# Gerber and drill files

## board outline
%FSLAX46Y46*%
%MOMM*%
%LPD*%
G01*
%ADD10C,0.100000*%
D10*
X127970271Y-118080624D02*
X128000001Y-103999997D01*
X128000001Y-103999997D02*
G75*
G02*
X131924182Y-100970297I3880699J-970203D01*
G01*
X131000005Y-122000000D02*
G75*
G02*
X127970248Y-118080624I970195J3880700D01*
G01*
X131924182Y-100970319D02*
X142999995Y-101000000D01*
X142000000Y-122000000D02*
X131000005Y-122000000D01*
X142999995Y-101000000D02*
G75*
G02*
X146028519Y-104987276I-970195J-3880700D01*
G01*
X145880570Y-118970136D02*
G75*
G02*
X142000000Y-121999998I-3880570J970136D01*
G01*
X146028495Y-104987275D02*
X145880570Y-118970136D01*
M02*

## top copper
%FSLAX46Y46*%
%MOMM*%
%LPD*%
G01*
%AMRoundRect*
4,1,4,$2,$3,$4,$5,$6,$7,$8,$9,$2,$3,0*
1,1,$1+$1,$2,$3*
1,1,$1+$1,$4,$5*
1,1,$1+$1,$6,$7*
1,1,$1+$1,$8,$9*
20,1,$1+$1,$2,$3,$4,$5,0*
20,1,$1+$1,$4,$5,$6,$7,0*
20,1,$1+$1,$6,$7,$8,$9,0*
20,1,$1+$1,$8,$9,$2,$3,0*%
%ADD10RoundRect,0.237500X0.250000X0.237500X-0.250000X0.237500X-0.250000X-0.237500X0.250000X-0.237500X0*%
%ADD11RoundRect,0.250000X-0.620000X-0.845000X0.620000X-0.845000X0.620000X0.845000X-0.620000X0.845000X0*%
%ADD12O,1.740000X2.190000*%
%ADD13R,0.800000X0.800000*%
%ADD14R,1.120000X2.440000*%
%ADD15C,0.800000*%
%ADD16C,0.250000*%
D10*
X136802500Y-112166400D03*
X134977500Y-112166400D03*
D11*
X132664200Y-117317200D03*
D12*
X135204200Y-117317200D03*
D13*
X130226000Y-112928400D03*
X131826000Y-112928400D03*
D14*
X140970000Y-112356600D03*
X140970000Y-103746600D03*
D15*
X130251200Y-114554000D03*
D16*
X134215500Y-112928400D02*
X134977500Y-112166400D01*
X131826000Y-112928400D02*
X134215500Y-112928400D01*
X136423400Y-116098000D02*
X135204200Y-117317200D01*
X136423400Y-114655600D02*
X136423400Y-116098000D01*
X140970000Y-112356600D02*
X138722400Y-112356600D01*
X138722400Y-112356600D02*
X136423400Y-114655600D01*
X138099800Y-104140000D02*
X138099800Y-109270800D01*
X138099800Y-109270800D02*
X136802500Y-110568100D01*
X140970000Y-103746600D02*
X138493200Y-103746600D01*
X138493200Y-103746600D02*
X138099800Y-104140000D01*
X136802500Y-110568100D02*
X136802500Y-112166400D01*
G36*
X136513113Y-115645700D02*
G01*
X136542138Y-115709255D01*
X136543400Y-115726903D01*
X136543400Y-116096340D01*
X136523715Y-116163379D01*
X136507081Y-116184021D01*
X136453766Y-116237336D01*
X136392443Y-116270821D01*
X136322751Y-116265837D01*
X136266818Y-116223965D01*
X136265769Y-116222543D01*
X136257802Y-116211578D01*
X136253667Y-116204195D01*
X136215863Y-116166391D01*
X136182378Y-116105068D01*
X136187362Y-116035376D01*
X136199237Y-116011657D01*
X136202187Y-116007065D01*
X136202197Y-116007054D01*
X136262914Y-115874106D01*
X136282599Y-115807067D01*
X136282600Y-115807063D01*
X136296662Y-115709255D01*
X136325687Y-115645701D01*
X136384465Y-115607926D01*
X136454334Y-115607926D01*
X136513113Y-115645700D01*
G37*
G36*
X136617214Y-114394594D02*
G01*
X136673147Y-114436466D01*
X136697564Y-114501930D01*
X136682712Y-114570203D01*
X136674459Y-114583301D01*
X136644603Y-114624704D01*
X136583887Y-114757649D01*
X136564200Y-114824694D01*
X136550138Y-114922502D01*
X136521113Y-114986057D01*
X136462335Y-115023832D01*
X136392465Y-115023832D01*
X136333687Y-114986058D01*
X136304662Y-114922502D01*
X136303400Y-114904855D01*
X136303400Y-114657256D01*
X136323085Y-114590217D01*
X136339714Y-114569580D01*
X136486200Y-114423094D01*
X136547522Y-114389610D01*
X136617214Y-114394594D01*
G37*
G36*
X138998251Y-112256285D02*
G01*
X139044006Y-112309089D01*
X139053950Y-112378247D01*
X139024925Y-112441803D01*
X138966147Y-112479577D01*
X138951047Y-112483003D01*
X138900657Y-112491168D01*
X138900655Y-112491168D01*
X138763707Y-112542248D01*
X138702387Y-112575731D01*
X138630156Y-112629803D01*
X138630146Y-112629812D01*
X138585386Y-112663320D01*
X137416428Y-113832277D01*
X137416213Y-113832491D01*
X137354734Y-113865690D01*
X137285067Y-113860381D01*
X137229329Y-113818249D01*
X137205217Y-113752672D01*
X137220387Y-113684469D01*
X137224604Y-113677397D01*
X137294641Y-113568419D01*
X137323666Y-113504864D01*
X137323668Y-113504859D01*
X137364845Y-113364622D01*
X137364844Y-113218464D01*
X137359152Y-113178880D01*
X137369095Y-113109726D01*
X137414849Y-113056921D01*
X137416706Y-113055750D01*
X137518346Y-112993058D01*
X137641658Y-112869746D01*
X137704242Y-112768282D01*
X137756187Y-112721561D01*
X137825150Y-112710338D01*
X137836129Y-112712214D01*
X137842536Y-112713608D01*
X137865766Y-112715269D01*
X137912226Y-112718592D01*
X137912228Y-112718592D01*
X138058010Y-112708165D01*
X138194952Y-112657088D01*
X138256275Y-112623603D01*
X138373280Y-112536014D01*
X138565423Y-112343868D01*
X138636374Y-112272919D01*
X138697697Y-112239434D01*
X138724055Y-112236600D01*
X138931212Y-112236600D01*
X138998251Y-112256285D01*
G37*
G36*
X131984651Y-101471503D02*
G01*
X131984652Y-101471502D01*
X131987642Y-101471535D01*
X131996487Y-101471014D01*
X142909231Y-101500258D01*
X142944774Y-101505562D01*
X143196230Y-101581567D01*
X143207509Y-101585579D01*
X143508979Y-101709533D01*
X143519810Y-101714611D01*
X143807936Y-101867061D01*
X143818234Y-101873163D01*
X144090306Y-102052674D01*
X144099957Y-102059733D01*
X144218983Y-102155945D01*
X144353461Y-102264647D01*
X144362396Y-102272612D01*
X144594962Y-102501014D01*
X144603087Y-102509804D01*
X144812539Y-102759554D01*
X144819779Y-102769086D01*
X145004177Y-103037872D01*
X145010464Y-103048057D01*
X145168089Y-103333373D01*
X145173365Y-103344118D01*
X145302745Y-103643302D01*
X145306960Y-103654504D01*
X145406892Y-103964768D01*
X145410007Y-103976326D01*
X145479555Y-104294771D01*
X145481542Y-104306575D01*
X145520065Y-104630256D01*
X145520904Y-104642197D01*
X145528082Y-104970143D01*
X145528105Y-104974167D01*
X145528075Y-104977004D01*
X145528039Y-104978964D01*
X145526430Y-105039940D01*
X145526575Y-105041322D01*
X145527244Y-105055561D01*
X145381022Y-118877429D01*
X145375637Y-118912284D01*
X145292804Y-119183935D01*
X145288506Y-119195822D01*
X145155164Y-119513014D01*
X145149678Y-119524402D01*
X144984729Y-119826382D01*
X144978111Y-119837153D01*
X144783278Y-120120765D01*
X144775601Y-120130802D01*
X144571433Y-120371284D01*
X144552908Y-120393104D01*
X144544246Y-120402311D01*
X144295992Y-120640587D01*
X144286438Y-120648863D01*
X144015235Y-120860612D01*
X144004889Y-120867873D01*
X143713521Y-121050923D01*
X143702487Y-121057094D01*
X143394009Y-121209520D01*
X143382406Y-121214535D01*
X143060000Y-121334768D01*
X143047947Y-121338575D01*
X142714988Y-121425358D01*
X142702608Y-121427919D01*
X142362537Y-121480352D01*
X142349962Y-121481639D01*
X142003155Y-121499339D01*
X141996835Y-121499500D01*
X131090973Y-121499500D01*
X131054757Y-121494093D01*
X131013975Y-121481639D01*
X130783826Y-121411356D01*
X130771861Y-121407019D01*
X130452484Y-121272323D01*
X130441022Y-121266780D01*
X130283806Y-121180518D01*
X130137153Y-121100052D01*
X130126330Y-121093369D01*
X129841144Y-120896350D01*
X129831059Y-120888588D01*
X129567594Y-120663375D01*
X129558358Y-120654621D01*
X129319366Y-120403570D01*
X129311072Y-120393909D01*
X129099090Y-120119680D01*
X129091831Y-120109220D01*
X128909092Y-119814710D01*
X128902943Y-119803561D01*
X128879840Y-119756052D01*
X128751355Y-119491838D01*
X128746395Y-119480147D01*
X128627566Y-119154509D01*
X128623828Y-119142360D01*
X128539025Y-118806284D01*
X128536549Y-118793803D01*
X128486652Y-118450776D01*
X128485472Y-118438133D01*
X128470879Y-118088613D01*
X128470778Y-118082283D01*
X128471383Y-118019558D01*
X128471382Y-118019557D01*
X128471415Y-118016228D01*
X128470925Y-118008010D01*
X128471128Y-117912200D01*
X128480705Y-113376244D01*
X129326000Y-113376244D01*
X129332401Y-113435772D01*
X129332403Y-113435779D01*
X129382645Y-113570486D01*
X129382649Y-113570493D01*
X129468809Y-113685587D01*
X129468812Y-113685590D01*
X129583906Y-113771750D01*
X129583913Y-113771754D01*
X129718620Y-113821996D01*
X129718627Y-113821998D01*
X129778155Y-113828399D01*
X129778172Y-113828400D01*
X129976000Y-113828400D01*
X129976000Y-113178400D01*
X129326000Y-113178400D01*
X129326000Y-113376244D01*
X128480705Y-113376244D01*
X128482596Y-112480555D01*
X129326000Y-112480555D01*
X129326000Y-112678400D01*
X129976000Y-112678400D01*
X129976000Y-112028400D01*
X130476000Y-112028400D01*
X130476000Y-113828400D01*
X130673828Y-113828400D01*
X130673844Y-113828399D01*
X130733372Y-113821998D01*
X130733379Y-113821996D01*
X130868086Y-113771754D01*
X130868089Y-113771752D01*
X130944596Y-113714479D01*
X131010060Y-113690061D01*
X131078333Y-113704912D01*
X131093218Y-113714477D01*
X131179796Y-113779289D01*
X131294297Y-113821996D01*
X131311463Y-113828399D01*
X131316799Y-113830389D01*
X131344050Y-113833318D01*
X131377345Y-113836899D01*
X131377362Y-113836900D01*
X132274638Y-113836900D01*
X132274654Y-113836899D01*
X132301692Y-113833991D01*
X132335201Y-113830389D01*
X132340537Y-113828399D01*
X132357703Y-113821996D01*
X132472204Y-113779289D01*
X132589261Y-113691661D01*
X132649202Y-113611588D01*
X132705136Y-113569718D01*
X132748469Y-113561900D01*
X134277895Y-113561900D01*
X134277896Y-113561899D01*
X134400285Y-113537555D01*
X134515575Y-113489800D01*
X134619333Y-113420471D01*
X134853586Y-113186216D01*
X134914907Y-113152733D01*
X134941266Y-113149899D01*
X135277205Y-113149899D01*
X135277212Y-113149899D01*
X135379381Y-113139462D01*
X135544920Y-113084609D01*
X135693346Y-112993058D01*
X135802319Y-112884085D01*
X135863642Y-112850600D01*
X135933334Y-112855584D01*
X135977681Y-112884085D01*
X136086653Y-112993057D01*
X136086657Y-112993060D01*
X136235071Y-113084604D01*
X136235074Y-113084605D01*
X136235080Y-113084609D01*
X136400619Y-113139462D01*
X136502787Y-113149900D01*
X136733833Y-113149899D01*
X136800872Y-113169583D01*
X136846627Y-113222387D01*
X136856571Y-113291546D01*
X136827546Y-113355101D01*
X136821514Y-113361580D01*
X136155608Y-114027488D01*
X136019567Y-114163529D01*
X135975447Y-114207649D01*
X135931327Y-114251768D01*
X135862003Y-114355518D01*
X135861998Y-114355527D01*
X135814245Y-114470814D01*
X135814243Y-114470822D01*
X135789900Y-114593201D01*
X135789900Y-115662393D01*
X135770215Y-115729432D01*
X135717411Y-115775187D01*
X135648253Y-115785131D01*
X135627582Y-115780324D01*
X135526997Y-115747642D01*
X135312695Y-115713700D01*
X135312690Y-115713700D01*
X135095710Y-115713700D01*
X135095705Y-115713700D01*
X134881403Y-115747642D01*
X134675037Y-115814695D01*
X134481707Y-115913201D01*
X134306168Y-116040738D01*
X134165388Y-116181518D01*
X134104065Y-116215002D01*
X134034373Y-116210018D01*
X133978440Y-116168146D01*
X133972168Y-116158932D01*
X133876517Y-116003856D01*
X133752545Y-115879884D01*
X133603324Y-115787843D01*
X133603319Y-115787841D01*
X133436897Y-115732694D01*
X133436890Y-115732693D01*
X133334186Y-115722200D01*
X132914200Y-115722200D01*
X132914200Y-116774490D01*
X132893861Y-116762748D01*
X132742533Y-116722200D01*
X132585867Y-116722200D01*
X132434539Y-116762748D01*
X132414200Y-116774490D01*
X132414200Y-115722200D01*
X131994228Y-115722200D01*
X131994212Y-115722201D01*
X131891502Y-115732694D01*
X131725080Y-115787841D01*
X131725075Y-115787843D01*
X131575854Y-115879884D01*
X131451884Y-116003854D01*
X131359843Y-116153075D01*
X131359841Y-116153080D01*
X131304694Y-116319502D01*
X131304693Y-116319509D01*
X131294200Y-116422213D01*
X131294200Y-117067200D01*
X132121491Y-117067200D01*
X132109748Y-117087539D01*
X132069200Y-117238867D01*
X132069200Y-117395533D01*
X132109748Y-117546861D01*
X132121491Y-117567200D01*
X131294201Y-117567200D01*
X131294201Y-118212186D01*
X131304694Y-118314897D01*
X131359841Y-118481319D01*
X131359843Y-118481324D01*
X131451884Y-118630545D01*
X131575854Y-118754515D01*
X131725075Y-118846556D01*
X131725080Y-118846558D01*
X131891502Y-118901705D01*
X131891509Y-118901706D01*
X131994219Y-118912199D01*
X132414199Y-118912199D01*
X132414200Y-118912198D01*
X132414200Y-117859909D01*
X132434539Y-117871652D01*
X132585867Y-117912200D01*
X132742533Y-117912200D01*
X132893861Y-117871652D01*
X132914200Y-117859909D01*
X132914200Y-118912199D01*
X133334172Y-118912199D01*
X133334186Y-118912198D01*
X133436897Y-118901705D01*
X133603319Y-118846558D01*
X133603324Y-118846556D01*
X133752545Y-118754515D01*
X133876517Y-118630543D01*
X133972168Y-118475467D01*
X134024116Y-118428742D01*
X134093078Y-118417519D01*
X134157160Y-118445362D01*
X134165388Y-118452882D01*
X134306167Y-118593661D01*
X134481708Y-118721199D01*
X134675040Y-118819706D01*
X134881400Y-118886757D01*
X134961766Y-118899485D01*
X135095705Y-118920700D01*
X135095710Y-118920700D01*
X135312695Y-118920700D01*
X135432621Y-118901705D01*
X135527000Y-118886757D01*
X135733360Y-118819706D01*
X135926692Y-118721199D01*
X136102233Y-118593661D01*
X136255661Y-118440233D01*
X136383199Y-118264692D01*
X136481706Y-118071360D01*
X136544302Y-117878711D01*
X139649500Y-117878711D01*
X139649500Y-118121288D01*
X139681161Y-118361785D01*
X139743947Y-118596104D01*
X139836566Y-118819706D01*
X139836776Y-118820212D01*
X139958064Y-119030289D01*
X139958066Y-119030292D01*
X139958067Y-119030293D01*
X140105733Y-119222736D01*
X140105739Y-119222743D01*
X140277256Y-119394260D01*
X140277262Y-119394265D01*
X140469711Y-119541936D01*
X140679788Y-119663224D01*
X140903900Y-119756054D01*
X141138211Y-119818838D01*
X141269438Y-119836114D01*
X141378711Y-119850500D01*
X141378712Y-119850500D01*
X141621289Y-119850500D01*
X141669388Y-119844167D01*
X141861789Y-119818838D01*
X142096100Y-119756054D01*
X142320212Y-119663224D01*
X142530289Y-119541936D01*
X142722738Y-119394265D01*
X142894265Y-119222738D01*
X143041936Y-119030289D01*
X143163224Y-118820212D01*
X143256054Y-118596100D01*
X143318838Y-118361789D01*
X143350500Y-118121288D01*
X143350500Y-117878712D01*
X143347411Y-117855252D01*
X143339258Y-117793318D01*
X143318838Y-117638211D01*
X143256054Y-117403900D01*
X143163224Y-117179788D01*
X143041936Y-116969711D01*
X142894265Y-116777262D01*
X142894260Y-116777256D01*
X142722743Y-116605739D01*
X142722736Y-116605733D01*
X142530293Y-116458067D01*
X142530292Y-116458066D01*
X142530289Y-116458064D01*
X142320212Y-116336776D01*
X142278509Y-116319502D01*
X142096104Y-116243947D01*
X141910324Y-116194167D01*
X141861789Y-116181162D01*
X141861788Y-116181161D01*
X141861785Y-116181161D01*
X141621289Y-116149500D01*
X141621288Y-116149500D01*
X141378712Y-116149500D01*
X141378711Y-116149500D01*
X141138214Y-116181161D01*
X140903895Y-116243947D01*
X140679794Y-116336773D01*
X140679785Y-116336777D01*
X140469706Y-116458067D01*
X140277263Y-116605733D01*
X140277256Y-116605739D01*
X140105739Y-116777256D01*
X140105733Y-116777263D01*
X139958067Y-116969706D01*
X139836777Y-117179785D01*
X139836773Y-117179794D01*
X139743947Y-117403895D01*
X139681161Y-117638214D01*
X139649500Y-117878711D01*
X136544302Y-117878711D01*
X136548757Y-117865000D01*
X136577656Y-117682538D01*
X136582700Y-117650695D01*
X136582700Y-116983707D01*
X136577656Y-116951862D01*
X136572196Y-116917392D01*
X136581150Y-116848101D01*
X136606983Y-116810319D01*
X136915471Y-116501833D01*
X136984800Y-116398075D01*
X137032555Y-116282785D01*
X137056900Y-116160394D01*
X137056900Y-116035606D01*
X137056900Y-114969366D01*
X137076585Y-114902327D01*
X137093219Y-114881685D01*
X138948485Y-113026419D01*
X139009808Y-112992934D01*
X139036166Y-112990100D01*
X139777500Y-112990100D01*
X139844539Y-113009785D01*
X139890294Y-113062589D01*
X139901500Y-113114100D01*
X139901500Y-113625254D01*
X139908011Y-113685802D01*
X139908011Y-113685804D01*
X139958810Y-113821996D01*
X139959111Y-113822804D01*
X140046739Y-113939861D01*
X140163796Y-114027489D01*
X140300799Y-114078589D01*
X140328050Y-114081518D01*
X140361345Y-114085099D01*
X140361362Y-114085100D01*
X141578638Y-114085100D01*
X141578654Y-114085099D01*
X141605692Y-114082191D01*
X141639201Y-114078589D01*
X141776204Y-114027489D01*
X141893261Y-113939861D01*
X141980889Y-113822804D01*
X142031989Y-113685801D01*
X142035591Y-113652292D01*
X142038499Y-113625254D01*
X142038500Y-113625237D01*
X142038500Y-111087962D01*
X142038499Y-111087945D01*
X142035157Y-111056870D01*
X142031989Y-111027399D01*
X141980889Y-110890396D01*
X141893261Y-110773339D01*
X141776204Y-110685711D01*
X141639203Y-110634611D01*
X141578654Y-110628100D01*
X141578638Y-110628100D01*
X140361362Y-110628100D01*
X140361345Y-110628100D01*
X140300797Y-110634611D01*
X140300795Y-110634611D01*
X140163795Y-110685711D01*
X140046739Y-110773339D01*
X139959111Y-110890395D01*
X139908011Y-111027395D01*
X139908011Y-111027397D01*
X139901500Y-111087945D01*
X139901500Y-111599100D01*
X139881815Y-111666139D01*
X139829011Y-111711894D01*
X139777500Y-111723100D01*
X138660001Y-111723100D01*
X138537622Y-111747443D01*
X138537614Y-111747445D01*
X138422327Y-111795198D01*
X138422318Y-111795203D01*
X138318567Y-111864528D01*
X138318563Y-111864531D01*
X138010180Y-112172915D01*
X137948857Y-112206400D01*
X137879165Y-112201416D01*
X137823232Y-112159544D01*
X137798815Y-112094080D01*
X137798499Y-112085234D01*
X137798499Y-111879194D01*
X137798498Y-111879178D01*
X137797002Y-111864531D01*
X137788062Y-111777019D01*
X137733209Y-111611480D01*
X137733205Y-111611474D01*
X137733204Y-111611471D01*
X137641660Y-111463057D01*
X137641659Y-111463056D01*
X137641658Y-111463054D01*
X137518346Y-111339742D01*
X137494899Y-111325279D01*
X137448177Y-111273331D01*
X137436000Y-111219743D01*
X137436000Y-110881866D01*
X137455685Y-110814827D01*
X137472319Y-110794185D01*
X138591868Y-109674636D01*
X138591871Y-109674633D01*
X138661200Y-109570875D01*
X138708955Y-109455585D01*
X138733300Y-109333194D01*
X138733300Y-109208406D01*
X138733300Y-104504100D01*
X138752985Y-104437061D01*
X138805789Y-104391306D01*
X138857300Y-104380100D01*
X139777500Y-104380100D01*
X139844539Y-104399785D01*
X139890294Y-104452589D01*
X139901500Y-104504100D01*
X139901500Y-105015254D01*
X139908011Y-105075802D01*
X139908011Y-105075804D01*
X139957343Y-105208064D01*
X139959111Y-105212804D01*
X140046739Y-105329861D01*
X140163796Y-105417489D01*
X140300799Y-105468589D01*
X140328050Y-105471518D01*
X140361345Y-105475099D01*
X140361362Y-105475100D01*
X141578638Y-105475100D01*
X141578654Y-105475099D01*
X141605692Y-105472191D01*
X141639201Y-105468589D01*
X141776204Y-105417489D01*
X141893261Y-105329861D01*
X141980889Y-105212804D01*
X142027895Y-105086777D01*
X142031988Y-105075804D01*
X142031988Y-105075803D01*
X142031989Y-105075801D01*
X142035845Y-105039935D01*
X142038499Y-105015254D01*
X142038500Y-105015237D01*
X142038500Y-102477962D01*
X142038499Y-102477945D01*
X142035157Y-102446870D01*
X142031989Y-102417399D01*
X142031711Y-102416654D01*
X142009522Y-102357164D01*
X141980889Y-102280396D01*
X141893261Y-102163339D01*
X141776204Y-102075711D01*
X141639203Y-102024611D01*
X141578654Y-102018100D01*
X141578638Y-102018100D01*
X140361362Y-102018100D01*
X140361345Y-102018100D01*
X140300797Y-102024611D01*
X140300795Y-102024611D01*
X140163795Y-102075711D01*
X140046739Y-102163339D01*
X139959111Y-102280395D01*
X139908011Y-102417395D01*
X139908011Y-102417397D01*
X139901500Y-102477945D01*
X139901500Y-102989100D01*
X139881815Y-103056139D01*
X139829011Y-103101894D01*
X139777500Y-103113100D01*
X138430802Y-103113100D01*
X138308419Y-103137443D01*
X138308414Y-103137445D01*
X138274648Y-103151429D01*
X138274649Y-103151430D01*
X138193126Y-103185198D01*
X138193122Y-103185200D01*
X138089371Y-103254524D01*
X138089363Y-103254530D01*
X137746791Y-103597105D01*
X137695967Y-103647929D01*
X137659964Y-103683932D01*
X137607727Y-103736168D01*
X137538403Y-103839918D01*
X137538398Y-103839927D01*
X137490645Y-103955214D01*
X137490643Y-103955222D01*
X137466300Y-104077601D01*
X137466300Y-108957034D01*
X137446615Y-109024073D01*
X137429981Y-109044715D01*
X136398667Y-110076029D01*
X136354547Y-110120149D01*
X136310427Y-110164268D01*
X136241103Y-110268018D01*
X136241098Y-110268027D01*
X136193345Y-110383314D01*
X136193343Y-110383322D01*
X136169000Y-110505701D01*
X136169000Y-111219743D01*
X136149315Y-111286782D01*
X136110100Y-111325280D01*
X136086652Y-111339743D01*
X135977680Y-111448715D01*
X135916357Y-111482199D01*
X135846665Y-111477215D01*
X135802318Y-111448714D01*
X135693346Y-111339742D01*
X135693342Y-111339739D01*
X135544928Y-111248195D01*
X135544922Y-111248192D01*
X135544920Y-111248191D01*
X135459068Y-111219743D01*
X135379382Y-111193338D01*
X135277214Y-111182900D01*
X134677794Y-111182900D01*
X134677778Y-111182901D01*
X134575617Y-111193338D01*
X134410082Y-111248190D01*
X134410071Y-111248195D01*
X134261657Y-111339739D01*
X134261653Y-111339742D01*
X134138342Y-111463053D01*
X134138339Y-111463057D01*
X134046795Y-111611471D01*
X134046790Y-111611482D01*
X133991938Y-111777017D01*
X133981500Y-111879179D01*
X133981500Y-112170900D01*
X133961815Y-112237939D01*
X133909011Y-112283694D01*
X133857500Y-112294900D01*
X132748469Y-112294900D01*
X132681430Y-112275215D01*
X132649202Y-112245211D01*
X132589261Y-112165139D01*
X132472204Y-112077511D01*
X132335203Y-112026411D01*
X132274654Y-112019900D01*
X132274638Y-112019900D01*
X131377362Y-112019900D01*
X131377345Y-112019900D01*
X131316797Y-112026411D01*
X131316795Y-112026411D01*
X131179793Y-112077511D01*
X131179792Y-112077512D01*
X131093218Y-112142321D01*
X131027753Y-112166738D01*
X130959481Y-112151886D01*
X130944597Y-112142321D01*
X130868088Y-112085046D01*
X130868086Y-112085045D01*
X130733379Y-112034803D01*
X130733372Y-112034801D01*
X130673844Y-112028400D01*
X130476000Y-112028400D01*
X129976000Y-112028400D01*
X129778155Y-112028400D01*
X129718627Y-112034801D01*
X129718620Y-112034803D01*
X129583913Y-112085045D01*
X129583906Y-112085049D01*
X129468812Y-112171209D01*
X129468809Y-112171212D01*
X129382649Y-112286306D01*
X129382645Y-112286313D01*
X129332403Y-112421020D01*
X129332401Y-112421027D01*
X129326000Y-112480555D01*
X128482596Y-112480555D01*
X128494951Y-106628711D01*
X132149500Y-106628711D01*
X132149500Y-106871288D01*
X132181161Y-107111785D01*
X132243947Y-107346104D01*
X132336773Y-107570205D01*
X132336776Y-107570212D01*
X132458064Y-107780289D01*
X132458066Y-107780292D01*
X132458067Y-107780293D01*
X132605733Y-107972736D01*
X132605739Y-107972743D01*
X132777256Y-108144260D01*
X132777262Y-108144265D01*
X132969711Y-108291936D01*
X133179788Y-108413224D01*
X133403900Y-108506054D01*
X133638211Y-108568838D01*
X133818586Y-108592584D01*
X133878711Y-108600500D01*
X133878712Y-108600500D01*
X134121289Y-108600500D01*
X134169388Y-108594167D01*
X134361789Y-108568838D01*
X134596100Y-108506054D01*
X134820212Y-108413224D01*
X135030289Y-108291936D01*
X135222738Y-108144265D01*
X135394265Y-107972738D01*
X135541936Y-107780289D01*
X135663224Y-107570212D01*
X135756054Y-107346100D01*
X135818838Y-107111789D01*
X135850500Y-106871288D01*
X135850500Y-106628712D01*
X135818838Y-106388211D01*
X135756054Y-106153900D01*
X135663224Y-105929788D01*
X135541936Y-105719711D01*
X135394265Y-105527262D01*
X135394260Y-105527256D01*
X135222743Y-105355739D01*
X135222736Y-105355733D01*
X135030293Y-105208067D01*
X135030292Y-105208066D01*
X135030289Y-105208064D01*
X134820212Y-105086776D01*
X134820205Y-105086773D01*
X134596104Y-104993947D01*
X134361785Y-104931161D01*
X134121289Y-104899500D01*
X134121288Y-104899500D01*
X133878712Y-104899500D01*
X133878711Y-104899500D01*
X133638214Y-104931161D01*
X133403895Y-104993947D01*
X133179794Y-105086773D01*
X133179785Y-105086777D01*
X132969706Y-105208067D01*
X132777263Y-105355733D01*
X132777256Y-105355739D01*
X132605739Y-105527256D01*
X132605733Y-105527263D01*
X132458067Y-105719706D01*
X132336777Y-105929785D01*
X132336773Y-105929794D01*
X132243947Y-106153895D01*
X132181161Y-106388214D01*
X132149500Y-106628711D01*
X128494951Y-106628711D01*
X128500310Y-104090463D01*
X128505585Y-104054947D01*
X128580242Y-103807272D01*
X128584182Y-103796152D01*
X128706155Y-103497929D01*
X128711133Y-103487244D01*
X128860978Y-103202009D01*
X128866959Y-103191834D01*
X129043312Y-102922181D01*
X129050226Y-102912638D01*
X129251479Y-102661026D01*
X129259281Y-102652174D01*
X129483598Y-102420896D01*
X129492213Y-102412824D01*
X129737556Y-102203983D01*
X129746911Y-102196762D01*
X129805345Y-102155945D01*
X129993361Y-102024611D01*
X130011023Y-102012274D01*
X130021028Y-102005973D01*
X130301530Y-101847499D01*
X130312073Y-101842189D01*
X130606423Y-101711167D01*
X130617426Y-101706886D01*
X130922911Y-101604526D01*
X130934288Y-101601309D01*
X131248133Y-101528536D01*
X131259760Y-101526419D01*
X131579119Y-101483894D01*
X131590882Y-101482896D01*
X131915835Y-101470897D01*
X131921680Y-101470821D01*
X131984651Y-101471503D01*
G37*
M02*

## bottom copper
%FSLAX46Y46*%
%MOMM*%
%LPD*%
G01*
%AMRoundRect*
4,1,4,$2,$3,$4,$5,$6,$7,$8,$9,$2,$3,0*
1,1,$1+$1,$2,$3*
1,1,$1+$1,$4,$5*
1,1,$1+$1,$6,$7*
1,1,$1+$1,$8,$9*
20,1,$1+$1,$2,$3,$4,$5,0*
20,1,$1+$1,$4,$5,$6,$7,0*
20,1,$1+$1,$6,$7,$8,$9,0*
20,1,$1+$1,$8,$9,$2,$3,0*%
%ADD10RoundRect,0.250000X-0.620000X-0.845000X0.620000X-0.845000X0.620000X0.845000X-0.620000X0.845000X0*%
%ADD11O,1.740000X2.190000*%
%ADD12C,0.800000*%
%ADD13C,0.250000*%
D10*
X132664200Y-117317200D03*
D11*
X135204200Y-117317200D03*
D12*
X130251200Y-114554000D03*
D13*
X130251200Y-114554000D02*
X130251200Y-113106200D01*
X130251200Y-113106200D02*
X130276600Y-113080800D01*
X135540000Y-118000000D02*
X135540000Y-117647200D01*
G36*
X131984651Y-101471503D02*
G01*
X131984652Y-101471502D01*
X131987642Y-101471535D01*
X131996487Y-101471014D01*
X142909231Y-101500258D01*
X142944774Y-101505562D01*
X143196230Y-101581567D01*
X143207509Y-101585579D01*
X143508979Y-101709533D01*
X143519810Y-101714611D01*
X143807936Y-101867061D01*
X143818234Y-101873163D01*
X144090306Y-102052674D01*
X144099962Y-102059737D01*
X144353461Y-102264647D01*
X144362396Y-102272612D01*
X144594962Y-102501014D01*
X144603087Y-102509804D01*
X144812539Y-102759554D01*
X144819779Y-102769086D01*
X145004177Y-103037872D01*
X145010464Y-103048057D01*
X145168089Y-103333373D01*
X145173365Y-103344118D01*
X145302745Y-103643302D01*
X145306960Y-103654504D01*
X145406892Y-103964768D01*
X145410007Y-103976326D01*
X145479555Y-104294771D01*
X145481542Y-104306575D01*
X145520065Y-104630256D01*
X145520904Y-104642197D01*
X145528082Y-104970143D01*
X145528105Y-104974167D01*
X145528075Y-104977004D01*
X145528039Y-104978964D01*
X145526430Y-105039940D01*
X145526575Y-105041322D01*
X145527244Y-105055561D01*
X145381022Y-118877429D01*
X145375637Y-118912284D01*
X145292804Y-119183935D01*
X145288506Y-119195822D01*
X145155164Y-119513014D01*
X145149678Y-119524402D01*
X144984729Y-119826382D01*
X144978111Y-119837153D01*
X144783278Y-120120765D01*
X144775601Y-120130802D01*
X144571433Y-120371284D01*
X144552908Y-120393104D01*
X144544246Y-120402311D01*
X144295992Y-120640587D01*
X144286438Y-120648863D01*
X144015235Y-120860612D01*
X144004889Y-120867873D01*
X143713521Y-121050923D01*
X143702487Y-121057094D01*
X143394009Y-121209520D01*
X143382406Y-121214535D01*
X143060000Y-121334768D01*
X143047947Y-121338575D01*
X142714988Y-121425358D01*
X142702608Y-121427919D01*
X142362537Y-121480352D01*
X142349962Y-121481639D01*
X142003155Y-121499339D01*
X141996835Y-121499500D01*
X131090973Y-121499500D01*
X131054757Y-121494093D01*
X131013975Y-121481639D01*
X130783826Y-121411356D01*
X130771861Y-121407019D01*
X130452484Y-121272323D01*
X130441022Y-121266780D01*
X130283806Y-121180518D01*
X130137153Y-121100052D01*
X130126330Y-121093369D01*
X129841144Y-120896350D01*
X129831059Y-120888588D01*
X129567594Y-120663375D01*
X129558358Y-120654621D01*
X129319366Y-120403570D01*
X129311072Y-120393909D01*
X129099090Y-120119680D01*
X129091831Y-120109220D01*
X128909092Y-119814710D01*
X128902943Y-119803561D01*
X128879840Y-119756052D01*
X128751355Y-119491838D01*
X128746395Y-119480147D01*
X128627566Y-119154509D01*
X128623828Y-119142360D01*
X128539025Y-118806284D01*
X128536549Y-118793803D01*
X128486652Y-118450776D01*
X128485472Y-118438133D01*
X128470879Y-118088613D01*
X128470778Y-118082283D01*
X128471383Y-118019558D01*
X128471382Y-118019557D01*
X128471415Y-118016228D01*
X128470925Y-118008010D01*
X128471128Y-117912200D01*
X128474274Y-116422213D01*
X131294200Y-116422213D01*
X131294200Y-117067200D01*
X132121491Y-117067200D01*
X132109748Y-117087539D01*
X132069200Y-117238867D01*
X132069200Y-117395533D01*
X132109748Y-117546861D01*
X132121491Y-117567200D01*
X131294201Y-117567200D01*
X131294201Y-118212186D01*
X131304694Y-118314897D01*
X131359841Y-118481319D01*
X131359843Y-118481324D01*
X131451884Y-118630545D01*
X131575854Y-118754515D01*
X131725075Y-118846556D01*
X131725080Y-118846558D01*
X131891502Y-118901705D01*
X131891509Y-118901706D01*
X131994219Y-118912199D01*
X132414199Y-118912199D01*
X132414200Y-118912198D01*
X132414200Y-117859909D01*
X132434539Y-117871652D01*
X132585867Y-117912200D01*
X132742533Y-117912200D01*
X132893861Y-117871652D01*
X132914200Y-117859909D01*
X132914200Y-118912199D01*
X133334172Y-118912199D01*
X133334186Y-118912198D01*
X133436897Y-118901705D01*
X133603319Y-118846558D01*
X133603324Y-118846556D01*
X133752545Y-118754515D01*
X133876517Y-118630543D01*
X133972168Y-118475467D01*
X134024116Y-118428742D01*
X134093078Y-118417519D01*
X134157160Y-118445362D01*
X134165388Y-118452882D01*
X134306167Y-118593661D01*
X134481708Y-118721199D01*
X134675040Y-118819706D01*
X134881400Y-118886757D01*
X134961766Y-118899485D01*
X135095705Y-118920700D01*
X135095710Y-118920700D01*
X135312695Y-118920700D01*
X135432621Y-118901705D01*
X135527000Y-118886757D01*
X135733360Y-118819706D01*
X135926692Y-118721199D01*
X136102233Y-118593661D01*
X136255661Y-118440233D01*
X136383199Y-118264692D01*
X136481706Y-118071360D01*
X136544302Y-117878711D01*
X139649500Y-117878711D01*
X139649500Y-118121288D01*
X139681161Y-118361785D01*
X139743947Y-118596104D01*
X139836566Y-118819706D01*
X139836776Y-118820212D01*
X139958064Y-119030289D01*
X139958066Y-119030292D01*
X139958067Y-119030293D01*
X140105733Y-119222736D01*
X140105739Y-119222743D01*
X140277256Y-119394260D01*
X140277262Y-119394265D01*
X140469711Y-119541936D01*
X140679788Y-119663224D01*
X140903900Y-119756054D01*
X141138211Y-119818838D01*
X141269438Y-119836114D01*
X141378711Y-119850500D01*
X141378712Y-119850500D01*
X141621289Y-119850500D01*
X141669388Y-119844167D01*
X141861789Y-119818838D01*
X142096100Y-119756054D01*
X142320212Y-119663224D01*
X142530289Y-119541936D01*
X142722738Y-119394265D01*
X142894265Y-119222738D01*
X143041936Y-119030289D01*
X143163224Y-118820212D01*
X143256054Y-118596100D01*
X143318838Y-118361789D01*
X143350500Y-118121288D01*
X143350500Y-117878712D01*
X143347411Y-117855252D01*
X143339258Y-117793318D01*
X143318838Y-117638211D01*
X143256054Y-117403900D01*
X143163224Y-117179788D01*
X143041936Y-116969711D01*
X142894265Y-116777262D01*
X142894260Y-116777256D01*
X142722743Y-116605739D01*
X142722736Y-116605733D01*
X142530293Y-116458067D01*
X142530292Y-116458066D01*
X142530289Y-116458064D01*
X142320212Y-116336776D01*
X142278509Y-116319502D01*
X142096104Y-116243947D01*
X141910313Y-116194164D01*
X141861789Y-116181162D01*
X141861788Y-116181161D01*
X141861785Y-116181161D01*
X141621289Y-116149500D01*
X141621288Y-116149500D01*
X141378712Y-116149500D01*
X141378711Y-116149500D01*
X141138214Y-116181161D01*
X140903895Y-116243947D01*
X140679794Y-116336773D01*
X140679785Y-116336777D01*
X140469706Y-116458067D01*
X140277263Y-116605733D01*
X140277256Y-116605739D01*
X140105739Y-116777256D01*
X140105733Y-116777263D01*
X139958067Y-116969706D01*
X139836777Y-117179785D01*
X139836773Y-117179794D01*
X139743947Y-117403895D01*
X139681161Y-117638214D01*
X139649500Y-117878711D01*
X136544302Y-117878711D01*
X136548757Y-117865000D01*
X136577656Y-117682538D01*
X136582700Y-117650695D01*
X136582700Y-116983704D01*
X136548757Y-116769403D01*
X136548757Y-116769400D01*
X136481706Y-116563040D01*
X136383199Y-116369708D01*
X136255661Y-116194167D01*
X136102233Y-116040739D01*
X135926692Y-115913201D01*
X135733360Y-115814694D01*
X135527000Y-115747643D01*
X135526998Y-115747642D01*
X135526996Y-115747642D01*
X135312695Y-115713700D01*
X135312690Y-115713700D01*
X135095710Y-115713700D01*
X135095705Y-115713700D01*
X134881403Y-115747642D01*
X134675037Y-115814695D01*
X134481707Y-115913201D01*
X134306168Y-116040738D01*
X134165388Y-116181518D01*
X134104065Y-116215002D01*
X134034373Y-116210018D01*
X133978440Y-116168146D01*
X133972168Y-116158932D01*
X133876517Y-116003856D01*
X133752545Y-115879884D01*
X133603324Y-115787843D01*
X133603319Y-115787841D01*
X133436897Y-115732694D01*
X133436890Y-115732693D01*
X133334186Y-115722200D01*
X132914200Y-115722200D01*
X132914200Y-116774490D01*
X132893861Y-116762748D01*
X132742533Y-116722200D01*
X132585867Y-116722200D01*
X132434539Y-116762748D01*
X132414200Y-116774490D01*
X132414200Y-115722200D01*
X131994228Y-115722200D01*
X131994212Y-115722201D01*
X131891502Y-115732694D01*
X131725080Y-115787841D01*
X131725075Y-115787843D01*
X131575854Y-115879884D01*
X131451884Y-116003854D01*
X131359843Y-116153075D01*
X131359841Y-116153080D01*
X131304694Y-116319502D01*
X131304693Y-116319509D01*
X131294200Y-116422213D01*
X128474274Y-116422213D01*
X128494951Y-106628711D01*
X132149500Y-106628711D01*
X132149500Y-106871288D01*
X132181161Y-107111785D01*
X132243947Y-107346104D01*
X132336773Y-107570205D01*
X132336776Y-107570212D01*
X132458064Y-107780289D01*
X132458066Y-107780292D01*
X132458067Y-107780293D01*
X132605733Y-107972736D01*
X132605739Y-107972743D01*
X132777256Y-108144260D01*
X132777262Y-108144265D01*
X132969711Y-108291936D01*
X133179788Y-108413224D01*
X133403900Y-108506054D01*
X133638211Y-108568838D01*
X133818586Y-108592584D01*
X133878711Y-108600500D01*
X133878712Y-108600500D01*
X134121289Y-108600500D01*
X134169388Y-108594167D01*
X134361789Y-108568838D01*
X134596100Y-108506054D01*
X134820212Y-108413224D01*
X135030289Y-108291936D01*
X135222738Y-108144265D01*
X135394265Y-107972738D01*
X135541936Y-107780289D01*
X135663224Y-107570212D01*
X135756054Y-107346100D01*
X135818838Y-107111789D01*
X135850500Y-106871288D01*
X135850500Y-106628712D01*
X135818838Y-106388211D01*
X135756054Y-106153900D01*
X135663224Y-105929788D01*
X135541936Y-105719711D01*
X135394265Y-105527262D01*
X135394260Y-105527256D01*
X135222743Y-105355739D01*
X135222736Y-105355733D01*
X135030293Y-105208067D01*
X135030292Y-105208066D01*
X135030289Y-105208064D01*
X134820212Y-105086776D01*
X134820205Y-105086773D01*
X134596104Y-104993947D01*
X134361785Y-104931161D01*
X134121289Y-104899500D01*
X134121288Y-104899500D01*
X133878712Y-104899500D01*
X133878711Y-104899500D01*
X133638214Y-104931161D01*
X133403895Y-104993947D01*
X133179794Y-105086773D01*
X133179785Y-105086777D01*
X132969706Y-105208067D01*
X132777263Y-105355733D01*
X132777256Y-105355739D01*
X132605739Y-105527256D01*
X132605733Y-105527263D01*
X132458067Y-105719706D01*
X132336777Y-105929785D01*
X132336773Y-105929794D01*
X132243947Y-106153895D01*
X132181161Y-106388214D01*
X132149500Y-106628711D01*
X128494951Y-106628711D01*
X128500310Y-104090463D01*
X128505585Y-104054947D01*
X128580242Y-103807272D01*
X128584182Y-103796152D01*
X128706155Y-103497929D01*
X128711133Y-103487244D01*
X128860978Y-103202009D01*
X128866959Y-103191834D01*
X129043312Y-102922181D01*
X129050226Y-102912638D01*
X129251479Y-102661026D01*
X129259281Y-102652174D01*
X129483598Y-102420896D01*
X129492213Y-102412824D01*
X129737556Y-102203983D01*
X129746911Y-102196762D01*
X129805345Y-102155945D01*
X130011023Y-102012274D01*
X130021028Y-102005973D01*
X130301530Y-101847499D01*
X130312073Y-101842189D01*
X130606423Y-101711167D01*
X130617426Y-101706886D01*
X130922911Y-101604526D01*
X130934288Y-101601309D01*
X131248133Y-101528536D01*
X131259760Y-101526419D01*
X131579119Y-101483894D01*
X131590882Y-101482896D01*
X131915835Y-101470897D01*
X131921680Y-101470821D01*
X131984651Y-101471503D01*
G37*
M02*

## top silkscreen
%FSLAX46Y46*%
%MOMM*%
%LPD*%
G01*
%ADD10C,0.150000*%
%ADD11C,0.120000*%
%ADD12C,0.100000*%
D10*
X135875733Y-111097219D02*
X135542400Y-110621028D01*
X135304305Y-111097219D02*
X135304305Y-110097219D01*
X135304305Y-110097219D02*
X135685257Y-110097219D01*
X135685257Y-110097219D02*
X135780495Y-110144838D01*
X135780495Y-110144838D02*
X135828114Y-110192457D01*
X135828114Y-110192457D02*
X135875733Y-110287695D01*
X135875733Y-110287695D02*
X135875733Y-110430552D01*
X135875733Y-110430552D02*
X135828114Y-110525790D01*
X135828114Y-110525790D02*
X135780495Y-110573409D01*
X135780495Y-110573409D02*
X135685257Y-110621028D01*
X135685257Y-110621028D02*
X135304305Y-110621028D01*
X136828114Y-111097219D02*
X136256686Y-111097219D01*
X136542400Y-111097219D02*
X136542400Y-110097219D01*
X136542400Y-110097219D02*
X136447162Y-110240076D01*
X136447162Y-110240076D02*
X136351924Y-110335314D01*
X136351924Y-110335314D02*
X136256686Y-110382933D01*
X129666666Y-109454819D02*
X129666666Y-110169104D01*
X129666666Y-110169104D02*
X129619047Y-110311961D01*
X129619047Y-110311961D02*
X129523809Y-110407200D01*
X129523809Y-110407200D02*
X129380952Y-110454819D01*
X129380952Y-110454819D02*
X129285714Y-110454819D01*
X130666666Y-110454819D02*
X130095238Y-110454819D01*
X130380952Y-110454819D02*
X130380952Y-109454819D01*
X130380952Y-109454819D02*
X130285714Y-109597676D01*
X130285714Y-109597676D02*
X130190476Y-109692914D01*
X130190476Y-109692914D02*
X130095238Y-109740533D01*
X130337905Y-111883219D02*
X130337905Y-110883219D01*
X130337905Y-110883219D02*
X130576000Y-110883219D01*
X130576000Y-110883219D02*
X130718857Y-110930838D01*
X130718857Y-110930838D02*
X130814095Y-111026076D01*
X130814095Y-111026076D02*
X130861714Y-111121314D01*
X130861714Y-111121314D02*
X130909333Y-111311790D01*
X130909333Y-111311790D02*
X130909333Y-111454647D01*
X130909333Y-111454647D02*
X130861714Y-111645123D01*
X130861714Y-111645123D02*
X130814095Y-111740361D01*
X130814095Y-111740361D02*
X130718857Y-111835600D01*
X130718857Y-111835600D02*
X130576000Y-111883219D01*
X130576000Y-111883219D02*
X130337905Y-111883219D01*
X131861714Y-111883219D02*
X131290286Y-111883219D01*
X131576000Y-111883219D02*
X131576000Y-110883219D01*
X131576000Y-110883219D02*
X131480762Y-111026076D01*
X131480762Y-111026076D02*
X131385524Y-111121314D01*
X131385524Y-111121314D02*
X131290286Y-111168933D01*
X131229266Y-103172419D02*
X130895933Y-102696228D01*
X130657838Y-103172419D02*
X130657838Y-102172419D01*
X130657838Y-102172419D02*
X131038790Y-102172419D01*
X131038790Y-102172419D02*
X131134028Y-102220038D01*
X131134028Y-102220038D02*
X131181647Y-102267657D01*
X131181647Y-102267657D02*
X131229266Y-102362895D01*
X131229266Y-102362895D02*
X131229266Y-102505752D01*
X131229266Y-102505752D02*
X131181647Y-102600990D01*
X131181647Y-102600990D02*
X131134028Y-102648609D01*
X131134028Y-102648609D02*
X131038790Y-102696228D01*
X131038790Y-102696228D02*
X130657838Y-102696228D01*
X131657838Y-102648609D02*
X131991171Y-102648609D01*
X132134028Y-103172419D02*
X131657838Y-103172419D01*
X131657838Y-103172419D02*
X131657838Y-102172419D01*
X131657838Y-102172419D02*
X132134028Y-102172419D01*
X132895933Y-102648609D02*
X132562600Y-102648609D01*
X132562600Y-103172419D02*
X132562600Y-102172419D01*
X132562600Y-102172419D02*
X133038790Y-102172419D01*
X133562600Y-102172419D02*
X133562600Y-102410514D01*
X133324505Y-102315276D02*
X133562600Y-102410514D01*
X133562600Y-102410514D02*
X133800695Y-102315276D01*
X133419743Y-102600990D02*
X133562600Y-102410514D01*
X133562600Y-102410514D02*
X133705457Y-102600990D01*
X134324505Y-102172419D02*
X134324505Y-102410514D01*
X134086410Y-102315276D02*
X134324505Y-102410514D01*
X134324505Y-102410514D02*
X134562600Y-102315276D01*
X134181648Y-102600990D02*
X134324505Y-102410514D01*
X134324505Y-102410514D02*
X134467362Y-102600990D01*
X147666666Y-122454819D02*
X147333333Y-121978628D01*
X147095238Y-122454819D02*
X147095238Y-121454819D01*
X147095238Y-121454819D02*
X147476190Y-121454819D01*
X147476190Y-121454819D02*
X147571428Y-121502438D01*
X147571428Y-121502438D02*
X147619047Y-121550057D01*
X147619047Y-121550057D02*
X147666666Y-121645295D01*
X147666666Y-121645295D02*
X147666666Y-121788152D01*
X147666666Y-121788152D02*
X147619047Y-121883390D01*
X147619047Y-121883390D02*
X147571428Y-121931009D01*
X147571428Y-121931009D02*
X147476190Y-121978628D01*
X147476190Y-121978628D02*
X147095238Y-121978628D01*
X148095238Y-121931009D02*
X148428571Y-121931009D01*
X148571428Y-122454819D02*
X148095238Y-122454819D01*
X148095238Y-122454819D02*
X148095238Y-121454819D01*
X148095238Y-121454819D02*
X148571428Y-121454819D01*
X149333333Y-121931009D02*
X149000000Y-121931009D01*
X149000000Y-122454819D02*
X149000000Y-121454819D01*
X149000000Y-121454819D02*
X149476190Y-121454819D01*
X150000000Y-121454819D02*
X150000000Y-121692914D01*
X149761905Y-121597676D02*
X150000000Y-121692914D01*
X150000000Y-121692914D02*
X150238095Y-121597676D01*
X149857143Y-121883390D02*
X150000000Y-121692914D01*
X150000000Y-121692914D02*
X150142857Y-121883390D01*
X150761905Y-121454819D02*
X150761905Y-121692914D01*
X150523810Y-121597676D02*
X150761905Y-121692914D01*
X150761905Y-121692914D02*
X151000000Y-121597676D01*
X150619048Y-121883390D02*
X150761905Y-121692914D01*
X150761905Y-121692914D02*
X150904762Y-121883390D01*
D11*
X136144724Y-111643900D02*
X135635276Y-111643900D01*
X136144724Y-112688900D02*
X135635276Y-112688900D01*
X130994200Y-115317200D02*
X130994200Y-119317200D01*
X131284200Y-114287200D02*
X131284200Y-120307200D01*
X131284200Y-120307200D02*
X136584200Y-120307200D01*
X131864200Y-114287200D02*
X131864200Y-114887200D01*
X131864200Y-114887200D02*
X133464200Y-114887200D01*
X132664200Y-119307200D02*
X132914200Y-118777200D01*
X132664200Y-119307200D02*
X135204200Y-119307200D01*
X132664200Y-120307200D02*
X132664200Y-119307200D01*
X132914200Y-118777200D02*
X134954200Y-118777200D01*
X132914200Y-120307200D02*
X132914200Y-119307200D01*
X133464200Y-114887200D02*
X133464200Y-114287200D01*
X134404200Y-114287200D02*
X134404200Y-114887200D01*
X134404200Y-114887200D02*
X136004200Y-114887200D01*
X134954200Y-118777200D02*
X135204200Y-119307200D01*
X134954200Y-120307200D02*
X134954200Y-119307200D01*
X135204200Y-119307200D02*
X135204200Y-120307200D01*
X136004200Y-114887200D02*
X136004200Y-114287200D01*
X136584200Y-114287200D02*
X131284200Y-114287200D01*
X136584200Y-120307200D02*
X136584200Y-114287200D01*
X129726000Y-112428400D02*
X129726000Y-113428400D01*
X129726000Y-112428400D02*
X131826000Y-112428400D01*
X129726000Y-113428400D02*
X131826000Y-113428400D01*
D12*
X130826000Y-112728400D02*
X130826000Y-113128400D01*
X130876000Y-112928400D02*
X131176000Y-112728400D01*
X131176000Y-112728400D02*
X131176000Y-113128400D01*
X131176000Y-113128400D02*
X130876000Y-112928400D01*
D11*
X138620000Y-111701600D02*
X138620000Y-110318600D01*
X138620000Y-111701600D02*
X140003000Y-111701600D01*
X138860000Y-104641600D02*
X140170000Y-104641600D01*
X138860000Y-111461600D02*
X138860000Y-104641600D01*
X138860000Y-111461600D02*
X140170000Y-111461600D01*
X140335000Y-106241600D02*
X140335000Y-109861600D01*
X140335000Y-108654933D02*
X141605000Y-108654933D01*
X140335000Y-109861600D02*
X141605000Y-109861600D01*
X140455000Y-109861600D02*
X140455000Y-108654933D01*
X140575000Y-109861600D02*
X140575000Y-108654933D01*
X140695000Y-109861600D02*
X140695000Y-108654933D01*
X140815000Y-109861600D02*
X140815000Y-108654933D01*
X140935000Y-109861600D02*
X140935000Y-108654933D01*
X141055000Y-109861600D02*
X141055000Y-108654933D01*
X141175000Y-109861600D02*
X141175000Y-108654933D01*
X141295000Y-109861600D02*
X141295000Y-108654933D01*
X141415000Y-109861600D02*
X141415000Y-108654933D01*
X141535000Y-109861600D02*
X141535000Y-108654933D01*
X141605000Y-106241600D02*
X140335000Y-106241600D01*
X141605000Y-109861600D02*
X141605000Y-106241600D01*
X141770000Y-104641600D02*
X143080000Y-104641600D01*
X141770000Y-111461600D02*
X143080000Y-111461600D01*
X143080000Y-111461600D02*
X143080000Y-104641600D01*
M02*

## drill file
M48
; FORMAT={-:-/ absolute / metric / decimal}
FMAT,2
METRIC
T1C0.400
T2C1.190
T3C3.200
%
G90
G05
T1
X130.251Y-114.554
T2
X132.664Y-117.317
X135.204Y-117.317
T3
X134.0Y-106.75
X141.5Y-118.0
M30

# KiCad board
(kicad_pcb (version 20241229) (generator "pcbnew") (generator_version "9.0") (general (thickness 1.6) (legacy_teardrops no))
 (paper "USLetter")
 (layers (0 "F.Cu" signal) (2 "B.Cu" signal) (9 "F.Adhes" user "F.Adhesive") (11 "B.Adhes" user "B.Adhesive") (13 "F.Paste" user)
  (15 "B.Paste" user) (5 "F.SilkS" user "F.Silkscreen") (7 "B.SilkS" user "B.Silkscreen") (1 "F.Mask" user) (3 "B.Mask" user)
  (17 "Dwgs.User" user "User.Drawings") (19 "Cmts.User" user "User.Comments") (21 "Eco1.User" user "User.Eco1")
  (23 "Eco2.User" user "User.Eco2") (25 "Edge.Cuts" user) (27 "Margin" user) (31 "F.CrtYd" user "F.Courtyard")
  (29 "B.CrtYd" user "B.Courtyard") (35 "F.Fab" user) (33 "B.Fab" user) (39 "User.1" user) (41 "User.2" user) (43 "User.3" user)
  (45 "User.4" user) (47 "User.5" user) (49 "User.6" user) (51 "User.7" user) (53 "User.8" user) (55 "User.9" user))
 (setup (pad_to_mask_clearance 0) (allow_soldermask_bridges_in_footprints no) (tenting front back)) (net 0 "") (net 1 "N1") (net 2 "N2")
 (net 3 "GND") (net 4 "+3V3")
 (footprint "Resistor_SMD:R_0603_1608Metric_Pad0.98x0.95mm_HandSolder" (layer "F.Cu") (at 135.89 112.1664 180)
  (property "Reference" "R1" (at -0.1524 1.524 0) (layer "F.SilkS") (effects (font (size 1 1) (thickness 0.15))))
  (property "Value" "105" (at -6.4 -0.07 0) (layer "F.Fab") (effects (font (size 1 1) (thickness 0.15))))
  (fp_line (start -0.254724 0.5225) (end 0.254724 0.5225) (stroke (width 0.12) (type solid)) (layer "F.SilkS"))
  (fp_line (start -0.254724 -0.5225) (end 0.254724 -0.5225) (stroke (width 0.12) (type solid)) (layer "F.SilkS"))
  (pad "1" smd roundrect (at -0.9125 0 180) (size 0.975 0.95) (layers "F.Cu" "F.Mask" "F.Paste") (roundrect_rratio 0.25) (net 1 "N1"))
  (pad "2" smd roundrect (at 0.9125 0 180) (size 0.975 0.95) (layers "F.Cu" "F.Mask" "F.Paste") (roundrect_rratio 0.25) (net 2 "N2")))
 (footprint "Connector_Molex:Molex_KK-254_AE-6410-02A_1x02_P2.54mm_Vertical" (layer "F.Cu") (at 132.6642 117.3172)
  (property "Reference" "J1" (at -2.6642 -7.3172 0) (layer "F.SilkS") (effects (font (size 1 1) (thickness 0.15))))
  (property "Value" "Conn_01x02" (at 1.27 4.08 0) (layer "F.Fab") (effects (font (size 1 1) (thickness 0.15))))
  (fp_line (start -1.67 -2) (end -1.67 2) (stroke (width 0.12) (type solid)) (layer "F.SilkS"))
  (fp_line (start -1.38 -3.03) (end -1.38 2.99) (stroke (width 0.12) (type solid)) (layer "F.SilkS"))
  (fp_line (start -1.38 2.99) (end 3.92 2.99) (stroke (width 0.12) (type solid)) (layer "F.SilkS"))
  (fp_line (start -0.8 -3.03) (end -0.8 -2.43) (stroke (width 0.12) (type solid)) (layer "F.SilkS"))
  (fp_line (start -0.8 -2.43) (end 0.8 -2.43) (stroke (width 0.12) (type solid)) (layer "F.SilkS"))
  (fp_line (start 0 1.99) (end 0.25 1.46) (stroke (width 0.12) (type solid)) (layer "F.SilkS"))
  (fp_line (start 0 1.99) (end 2.54 1.99) (stroke (width 0.12) (type solid)) (layer "F.SilkS"))
  (fp_line (start 0 2.99) (end 0 1.99) (stroke (width 0.12) (type solid)) (layer "F.SilkS"))
  (fp_line (start 0.25 1.46) (end 2.29 1.46) (stroke (width 0.12) (type solid)) (layer "F.SilkS"))
  (fp_line (start 0.25 2.99) (end 0.25 1.99) (stroke (width 0.12) (type solid)) (layer "F.SilkS"))
  (fp_line (start 0.8 -2.43) (end 0.8 -3.03) (stroke (width 0.12) (type solid)) (layer "F.SilkS"))
  (fp_line (start 1.74 -3.03) (end 1.74 -2.43) (stroke (width 0.12) (type solid)) (layer "F.SilkS"))
  (fp_line (start 1.74 -2.43) (end 3.34 -2.43) (stroke (width 0.12) (type solid)) (layer "F.SilkS"))
  (fp_line (start 2.29 1.46) (end 2.54 1.99) (stroke (width 0.12) (type solid)) (layer "F.SilkS"))
  (fp_line (start 2.29 2.99) (end 2.29 1.99) (stroke (width 0.12) (type solid)) (layer "F.SilkS"))
  (fp_line (start 2.54 1.99) (end 2.54 2.99) (stroke (width 0.12) (type solid)) (layer "F.SilkS"))
  (fp_line (start 3.34 -2.43) (end 3.34 -3.03) (stroke (width 0.12) (type solid)) (layer "F.SilkS"))
  (fp_line (start 3.92 -3.03) (end -1.38 -3.03) (stroke (width 0.12) (type solid)) (layer "F.SilkS"))
  (fp_line (start 3.92 2.99) (end 3.92 -3.03) (stroke (width 0.12) (type solid)) (layer "F.SilkS"))
  (pad "1" thru_hole roundrect (at 0 0) (size 1.74 2.19) (drill 1.19) (layers "*.Cu" "*.Mask") (remove_unused_layers no)
   (roundrect_rratio 0.143678) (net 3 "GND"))
  (pad "2" thru_hole oval (at 2.54 0) (size 1.74 2.19) (drill 1.19) (layers "*.Cu" "*.Mask") (remove_unused_layers no) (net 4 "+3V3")))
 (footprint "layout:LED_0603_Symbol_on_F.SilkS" (layer "F.Cu") (at 131.026 112.9284)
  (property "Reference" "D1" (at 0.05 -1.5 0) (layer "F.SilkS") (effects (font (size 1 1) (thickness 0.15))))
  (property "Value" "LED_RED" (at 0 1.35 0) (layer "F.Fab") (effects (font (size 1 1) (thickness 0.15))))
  (fp_line (start -1.3 -0.5) (end -1.3 0.5) (stroke (width 0.12) (type solid)) (layer "F.SilkS"))
  (fp_line (start -1.3 -0.5) (end 0.8 -0.5) (stroke (width 0.12) (type solid)) (layer "F.SilkS"))
  (fp_line (start -1.3 0.5) (end 0.8 0.5) (stroke (width 0.12) (type solid)) (layer "F.SilkS"))
  (fp_line (start -0.2 -0.2) (end -0.2 0.2) (stroke (width 0.1) (type solid)) (layer "F.SilkS"))
  (fp_line (start -0.15 0) (end 0.15 -0.2) (stroke (width 0.1) (type solid)) (layer "F.SilkS"))
  (fp_line (start 0.15 -0.2) (end 0.15 0.2) (stroke (width 0.1) (type solid)) (layer "F.SilkS"))
  (fp_line (start 0.15 0.2) (end -0.15 0) (stroke (width 0.1) (type solid)) (layer "F.SilkS"))
  (pad "1" smd rect (at -0.8 0 180) (size 0.8 0.8) (layers "F.Cu" "F.Mask" "F.Paste") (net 3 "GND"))
  (pad "2" smd rect (at 0.8 0 180) (size 0.8 0.8) (layers "F.Cu" "F.Mask" "F.Paste") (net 2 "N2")))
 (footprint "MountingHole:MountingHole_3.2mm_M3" (layer "F.Cu") (at 134 106.75)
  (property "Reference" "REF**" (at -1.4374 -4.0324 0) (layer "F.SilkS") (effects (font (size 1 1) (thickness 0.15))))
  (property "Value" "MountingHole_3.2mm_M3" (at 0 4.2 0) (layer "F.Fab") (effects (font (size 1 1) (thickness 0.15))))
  (pad "" np_thru_hole circle (at 0 0) (size 3.2 3.2) (drill 3.2) (layers "*.Cu" "*.Mask")))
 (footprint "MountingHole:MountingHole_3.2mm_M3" (layer "F.Cu") (at 141.5 118)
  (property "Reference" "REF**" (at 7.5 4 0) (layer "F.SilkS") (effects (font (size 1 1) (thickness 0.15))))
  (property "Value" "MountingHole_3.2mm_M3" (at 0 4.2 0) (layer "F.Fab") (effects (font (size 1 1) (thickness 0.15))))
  (pad "" np_thru_hole circle (at 0 0) (size 3.2 3.2) (drill 3.2) (layers "*.Cu" "*.Mask")))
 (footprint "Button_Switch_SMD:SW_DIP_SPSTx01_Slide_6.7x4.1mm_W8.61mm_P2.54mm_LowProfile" (layer "F.Cu") (at 140.97 108.0516 90)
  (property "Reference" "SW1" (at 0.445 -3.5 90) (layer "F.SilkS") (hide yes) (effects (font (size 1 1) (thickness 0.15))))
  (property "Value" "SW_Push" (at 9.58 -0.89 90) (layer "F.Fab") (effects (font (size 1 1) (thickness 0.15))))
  (fp_line (start -3.65 -2.35) (end -2.267 -2.35) (stroke (width 0.12) (type solid)) (layer "F.SilkS"))
  (fp_line (start -3.65 -2.35) (end -3.65 -0.967) (stroke (width 0.12) (type solid)) (layer "F.SilkS"))
  (fp_line (start 3.41 -2.11) (end 3.41 -0.8) (stroke (width 0.12) (type solid)) (layer "F.SilkS"))
  (fp_line (start -3.41 -2.11) (end 3.41 -2.11) (stroke (width 0.12) (type solid)) (layer "F.SilkS"))
  (fp_line (start -3.41 -2.11) (end -3.41 -0.8) (stroke (width 0.12) (type solid)) (layer "F.SilkS"))
  (fp_line (start 1.81 -0.635) (end -1.81 -0.635) (stroke (width 0.12) (type solid)) (layer "F.SilkS"))
  (fp_line (start -0.603333 -0.635) (end -0.603333 0.635) (stroke (width 0.12) (type solid)) (layer "F.SilkS"))
  (fp_line (start -1.81 -0.635) (end -1.81 0.635) (stroke (width 0.12) (type solid)) (layer "F.SilkS"))
  (fp_line (start -1.81 -0.515) (end -0.603333 -0.515) (stroke (width 0.12) (type solid)) (layer "F.SilkS"))
  (fp_line (start -1.81 -0.395) (end -0.603333 -0.395) (stroke (width 0.12) (type solid)) (layer "F.SilkS"))
  (fp_line (start -1.81 -0.275) (end -0.603333 -0.275) (stroke (width 0.12) (type solid)) (layer "F.SilkS"))
  (fp_line (start -1.81 -0.155) (end -0.603333 -0.155) (stroke (width 0.12) (type solid)) (layer "F.SilkS"))
  (fp_line (start -1.81 -0.035) (end -0.603333 -0.035) (stroke (width 0.12) (type solid)) (layer "F.SilkS"))
  (fp_line (start -1.81 0.085) (end -0.603333 0.085) (stroke (width 0.12) (type solid)) (layer "F.SilkS"))
  (fp_line (start -1.81 0.205) (end -0.603333 0.205) (stroke (width 0.12) (type solid)) (layer "F.SilkS"))
  (fp_line (start -1.81 0.325) (end -0.603333 0.325) (stroke (width 0.12) (type solid)) (layer "F.SilkS"))
  (fp_line (start -1.81 0.445) (end -0.603333 0.445) (stroke (width 0.12) (type solid)) (layer "F.SilkS"))
  (fp_line (start -1.81 0.565) (end -0.603333 0.565) (stroke (width 0.12) (type solid)) (layer "F.SilkS"))
  (fp_line (start 1.81 0.635) (end 1.81 -0.635) (stroke (width 0.12) (type solid)) (layer "F.SilkS"))
  (fp_line (start -1.81 0.635) (end 1.81 0.635) (stroke (width 0.12) (type solid)) (layer "F.SilkS"))
  (fp_line (start 3.41 0.8) (end 3.41 2.11) (stroke (width 0.12) (type solid)) (layer "F.SilkS"))
  (fp_line (start -3.41 0.8) (end -3.41 2.11) (stroke (width 0.12) (type solid)) (layer "F.SilkS"))
  (fp_line (start -3.41 2.11) (end 3.41 2.11) (stroke (width 0.12) (type solid)) (layer "F.SilkS"))
  (pad "1" smd rect (at -4.305 0 90) (size 2.44 1.12) (layers "F.Cu" "F.Mask" "F.Paste") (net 4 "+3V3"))
  (pad "2" smd rect (at 4.305 0 90) (size 2.44 1.12) (layers "F.Cu" "F.Mask" "F.Paste") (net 1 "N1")))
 (gr_line (start 127.970271 118.080624) (end 128.000001 103.999997) (stroke (width 0.1) (type default)) (layer "Edge.Cuts"))
 (gr_arc (start 128.000001 103.999997) (mid 129.418921 101.817321) (end 131.924182 100.970319) (stroke (width 0.1) (type default))
  (layer "Edge.Cuts"))
 (gr_arc (start 131.000005 122) (mid 128.817321 120.581079) (end 127.970271 118.080624) (stroke (width 0.1) (type default))
  (layer "Edge.Cuts"))
 (gr_line (start 131.924182 100.970319) (end 142.999995 101) (stroke (width 0.1) (type default)) (layer "Edge.Cuts"))
 (gr_line (start 142 122) (end 131.000005 122) (stroke (width 0.1) (type default)) (layer "Edge.Cuts"))
 (gr_arc (start 142.999995 101) (mid 145.182679 102.418921) (end 146.028495 104.987275) (stroke (width 0.1) (type default))
  (layer "Edge.Cuts"))
 (gr_arc (start 145.88057 118.970136) (mid 144.461649 121.152822) (end 142 122) (stroke (width 0.1) (type default)) (layer "Edge.Cuts"))
 (gr_line (start 146.028495 104.987275) (end 145.88057 118.970136) (stroke (width 0.1) (type default)) (layer "Edge.Cuts"))
 (via (at 130.2512 114.554) (size 0.8) (drill 0.4) (layers "F.Cu" "B.Cu") (free yes) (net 3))
 (segment (start 130.2512 114.554) (end 130.2512 113.1062) (width 0.25) (layer "B.Cu") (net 3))
 (segment (start 130.2512 113.1062) (end 130.2766 113.0808) (width 0.25) (layer "B.Cu") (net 3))
 (segment (start 134.2155 112.9284) (end 134.9775 112.1664) (width 0.25) (layer "F.Cu") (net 2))
 (segment (start 131.826 112.9284) (end 134.2155 112.9284) (width 0.25) (layer "F.Cu") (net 2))
 (segment (start 136.4234 116.098) (end 135.2042 117.3172) (width 0.25) (layer "F.Cu") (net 4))
 (segment (start 136.4234 114.6556) (end 136.4234 116.098) (width 0.25) (layer "F.Cu") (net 4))
 (segment (start 140.97 112.3566) (end 138.7224 112.3566) (width 0.25) (layer "F.Cu") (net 4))
 (segment (start 138.7224 112.3566) (end 136.4234 114.6556) (width 0.25) (layer "F.Cu") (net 4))
 (segment (start 135.54 118) (end 135.54 117.6472) (width 0.25) (layer "B.Cu") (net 4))
 (segment (start 138.0998 104.14) (end 138.0998 109.2708) (width 0.25) (layer "F.Cu") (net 1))
 (segment (start 138.0998 109.2708) (end 136.8025 110.5681) (width 0.25) (layer "F.Cu") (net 1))
 (segment (start 140.97 103.7466) (end 138.4932 103.7466) (width 0.25) (layer "F.Cu") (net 1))
 (segment (start 138.4932 103.7466) (end 138.0998 104.14) (width 0.25) (layer "F.Cu") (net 1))
 (segment (start 136.8025 110.5681) (end 136.8025 112.1664) (width 0.25) (layer "F.Cu") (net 1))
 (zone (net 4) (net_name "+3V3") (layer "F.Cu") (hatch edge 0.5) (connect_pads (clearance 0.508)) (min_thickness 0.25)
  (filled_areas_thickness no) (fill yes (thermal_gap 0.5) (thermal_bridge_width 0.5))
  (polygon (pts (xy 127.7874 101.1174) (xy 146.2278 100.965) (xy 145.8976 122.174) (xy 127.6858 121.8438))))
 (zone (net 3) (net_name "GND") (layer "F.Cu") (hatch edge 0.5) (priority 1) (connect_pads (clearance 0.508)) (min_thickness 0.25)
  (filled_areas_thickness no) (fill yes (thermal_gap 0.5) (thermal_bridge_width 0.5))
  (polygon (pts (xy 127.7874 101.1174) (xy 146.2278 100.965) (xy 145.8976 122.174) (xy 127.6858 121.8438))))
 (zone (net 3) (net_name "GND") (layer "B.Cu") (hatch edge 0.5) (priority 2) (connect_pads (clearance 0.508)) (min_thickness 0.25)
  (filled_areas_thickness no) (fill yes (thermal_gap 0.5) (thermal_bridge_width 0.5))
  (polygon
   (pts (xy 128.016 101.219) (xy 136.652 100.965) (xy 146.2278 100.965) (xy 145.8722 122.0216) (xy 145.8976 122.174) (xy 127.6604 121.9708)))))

